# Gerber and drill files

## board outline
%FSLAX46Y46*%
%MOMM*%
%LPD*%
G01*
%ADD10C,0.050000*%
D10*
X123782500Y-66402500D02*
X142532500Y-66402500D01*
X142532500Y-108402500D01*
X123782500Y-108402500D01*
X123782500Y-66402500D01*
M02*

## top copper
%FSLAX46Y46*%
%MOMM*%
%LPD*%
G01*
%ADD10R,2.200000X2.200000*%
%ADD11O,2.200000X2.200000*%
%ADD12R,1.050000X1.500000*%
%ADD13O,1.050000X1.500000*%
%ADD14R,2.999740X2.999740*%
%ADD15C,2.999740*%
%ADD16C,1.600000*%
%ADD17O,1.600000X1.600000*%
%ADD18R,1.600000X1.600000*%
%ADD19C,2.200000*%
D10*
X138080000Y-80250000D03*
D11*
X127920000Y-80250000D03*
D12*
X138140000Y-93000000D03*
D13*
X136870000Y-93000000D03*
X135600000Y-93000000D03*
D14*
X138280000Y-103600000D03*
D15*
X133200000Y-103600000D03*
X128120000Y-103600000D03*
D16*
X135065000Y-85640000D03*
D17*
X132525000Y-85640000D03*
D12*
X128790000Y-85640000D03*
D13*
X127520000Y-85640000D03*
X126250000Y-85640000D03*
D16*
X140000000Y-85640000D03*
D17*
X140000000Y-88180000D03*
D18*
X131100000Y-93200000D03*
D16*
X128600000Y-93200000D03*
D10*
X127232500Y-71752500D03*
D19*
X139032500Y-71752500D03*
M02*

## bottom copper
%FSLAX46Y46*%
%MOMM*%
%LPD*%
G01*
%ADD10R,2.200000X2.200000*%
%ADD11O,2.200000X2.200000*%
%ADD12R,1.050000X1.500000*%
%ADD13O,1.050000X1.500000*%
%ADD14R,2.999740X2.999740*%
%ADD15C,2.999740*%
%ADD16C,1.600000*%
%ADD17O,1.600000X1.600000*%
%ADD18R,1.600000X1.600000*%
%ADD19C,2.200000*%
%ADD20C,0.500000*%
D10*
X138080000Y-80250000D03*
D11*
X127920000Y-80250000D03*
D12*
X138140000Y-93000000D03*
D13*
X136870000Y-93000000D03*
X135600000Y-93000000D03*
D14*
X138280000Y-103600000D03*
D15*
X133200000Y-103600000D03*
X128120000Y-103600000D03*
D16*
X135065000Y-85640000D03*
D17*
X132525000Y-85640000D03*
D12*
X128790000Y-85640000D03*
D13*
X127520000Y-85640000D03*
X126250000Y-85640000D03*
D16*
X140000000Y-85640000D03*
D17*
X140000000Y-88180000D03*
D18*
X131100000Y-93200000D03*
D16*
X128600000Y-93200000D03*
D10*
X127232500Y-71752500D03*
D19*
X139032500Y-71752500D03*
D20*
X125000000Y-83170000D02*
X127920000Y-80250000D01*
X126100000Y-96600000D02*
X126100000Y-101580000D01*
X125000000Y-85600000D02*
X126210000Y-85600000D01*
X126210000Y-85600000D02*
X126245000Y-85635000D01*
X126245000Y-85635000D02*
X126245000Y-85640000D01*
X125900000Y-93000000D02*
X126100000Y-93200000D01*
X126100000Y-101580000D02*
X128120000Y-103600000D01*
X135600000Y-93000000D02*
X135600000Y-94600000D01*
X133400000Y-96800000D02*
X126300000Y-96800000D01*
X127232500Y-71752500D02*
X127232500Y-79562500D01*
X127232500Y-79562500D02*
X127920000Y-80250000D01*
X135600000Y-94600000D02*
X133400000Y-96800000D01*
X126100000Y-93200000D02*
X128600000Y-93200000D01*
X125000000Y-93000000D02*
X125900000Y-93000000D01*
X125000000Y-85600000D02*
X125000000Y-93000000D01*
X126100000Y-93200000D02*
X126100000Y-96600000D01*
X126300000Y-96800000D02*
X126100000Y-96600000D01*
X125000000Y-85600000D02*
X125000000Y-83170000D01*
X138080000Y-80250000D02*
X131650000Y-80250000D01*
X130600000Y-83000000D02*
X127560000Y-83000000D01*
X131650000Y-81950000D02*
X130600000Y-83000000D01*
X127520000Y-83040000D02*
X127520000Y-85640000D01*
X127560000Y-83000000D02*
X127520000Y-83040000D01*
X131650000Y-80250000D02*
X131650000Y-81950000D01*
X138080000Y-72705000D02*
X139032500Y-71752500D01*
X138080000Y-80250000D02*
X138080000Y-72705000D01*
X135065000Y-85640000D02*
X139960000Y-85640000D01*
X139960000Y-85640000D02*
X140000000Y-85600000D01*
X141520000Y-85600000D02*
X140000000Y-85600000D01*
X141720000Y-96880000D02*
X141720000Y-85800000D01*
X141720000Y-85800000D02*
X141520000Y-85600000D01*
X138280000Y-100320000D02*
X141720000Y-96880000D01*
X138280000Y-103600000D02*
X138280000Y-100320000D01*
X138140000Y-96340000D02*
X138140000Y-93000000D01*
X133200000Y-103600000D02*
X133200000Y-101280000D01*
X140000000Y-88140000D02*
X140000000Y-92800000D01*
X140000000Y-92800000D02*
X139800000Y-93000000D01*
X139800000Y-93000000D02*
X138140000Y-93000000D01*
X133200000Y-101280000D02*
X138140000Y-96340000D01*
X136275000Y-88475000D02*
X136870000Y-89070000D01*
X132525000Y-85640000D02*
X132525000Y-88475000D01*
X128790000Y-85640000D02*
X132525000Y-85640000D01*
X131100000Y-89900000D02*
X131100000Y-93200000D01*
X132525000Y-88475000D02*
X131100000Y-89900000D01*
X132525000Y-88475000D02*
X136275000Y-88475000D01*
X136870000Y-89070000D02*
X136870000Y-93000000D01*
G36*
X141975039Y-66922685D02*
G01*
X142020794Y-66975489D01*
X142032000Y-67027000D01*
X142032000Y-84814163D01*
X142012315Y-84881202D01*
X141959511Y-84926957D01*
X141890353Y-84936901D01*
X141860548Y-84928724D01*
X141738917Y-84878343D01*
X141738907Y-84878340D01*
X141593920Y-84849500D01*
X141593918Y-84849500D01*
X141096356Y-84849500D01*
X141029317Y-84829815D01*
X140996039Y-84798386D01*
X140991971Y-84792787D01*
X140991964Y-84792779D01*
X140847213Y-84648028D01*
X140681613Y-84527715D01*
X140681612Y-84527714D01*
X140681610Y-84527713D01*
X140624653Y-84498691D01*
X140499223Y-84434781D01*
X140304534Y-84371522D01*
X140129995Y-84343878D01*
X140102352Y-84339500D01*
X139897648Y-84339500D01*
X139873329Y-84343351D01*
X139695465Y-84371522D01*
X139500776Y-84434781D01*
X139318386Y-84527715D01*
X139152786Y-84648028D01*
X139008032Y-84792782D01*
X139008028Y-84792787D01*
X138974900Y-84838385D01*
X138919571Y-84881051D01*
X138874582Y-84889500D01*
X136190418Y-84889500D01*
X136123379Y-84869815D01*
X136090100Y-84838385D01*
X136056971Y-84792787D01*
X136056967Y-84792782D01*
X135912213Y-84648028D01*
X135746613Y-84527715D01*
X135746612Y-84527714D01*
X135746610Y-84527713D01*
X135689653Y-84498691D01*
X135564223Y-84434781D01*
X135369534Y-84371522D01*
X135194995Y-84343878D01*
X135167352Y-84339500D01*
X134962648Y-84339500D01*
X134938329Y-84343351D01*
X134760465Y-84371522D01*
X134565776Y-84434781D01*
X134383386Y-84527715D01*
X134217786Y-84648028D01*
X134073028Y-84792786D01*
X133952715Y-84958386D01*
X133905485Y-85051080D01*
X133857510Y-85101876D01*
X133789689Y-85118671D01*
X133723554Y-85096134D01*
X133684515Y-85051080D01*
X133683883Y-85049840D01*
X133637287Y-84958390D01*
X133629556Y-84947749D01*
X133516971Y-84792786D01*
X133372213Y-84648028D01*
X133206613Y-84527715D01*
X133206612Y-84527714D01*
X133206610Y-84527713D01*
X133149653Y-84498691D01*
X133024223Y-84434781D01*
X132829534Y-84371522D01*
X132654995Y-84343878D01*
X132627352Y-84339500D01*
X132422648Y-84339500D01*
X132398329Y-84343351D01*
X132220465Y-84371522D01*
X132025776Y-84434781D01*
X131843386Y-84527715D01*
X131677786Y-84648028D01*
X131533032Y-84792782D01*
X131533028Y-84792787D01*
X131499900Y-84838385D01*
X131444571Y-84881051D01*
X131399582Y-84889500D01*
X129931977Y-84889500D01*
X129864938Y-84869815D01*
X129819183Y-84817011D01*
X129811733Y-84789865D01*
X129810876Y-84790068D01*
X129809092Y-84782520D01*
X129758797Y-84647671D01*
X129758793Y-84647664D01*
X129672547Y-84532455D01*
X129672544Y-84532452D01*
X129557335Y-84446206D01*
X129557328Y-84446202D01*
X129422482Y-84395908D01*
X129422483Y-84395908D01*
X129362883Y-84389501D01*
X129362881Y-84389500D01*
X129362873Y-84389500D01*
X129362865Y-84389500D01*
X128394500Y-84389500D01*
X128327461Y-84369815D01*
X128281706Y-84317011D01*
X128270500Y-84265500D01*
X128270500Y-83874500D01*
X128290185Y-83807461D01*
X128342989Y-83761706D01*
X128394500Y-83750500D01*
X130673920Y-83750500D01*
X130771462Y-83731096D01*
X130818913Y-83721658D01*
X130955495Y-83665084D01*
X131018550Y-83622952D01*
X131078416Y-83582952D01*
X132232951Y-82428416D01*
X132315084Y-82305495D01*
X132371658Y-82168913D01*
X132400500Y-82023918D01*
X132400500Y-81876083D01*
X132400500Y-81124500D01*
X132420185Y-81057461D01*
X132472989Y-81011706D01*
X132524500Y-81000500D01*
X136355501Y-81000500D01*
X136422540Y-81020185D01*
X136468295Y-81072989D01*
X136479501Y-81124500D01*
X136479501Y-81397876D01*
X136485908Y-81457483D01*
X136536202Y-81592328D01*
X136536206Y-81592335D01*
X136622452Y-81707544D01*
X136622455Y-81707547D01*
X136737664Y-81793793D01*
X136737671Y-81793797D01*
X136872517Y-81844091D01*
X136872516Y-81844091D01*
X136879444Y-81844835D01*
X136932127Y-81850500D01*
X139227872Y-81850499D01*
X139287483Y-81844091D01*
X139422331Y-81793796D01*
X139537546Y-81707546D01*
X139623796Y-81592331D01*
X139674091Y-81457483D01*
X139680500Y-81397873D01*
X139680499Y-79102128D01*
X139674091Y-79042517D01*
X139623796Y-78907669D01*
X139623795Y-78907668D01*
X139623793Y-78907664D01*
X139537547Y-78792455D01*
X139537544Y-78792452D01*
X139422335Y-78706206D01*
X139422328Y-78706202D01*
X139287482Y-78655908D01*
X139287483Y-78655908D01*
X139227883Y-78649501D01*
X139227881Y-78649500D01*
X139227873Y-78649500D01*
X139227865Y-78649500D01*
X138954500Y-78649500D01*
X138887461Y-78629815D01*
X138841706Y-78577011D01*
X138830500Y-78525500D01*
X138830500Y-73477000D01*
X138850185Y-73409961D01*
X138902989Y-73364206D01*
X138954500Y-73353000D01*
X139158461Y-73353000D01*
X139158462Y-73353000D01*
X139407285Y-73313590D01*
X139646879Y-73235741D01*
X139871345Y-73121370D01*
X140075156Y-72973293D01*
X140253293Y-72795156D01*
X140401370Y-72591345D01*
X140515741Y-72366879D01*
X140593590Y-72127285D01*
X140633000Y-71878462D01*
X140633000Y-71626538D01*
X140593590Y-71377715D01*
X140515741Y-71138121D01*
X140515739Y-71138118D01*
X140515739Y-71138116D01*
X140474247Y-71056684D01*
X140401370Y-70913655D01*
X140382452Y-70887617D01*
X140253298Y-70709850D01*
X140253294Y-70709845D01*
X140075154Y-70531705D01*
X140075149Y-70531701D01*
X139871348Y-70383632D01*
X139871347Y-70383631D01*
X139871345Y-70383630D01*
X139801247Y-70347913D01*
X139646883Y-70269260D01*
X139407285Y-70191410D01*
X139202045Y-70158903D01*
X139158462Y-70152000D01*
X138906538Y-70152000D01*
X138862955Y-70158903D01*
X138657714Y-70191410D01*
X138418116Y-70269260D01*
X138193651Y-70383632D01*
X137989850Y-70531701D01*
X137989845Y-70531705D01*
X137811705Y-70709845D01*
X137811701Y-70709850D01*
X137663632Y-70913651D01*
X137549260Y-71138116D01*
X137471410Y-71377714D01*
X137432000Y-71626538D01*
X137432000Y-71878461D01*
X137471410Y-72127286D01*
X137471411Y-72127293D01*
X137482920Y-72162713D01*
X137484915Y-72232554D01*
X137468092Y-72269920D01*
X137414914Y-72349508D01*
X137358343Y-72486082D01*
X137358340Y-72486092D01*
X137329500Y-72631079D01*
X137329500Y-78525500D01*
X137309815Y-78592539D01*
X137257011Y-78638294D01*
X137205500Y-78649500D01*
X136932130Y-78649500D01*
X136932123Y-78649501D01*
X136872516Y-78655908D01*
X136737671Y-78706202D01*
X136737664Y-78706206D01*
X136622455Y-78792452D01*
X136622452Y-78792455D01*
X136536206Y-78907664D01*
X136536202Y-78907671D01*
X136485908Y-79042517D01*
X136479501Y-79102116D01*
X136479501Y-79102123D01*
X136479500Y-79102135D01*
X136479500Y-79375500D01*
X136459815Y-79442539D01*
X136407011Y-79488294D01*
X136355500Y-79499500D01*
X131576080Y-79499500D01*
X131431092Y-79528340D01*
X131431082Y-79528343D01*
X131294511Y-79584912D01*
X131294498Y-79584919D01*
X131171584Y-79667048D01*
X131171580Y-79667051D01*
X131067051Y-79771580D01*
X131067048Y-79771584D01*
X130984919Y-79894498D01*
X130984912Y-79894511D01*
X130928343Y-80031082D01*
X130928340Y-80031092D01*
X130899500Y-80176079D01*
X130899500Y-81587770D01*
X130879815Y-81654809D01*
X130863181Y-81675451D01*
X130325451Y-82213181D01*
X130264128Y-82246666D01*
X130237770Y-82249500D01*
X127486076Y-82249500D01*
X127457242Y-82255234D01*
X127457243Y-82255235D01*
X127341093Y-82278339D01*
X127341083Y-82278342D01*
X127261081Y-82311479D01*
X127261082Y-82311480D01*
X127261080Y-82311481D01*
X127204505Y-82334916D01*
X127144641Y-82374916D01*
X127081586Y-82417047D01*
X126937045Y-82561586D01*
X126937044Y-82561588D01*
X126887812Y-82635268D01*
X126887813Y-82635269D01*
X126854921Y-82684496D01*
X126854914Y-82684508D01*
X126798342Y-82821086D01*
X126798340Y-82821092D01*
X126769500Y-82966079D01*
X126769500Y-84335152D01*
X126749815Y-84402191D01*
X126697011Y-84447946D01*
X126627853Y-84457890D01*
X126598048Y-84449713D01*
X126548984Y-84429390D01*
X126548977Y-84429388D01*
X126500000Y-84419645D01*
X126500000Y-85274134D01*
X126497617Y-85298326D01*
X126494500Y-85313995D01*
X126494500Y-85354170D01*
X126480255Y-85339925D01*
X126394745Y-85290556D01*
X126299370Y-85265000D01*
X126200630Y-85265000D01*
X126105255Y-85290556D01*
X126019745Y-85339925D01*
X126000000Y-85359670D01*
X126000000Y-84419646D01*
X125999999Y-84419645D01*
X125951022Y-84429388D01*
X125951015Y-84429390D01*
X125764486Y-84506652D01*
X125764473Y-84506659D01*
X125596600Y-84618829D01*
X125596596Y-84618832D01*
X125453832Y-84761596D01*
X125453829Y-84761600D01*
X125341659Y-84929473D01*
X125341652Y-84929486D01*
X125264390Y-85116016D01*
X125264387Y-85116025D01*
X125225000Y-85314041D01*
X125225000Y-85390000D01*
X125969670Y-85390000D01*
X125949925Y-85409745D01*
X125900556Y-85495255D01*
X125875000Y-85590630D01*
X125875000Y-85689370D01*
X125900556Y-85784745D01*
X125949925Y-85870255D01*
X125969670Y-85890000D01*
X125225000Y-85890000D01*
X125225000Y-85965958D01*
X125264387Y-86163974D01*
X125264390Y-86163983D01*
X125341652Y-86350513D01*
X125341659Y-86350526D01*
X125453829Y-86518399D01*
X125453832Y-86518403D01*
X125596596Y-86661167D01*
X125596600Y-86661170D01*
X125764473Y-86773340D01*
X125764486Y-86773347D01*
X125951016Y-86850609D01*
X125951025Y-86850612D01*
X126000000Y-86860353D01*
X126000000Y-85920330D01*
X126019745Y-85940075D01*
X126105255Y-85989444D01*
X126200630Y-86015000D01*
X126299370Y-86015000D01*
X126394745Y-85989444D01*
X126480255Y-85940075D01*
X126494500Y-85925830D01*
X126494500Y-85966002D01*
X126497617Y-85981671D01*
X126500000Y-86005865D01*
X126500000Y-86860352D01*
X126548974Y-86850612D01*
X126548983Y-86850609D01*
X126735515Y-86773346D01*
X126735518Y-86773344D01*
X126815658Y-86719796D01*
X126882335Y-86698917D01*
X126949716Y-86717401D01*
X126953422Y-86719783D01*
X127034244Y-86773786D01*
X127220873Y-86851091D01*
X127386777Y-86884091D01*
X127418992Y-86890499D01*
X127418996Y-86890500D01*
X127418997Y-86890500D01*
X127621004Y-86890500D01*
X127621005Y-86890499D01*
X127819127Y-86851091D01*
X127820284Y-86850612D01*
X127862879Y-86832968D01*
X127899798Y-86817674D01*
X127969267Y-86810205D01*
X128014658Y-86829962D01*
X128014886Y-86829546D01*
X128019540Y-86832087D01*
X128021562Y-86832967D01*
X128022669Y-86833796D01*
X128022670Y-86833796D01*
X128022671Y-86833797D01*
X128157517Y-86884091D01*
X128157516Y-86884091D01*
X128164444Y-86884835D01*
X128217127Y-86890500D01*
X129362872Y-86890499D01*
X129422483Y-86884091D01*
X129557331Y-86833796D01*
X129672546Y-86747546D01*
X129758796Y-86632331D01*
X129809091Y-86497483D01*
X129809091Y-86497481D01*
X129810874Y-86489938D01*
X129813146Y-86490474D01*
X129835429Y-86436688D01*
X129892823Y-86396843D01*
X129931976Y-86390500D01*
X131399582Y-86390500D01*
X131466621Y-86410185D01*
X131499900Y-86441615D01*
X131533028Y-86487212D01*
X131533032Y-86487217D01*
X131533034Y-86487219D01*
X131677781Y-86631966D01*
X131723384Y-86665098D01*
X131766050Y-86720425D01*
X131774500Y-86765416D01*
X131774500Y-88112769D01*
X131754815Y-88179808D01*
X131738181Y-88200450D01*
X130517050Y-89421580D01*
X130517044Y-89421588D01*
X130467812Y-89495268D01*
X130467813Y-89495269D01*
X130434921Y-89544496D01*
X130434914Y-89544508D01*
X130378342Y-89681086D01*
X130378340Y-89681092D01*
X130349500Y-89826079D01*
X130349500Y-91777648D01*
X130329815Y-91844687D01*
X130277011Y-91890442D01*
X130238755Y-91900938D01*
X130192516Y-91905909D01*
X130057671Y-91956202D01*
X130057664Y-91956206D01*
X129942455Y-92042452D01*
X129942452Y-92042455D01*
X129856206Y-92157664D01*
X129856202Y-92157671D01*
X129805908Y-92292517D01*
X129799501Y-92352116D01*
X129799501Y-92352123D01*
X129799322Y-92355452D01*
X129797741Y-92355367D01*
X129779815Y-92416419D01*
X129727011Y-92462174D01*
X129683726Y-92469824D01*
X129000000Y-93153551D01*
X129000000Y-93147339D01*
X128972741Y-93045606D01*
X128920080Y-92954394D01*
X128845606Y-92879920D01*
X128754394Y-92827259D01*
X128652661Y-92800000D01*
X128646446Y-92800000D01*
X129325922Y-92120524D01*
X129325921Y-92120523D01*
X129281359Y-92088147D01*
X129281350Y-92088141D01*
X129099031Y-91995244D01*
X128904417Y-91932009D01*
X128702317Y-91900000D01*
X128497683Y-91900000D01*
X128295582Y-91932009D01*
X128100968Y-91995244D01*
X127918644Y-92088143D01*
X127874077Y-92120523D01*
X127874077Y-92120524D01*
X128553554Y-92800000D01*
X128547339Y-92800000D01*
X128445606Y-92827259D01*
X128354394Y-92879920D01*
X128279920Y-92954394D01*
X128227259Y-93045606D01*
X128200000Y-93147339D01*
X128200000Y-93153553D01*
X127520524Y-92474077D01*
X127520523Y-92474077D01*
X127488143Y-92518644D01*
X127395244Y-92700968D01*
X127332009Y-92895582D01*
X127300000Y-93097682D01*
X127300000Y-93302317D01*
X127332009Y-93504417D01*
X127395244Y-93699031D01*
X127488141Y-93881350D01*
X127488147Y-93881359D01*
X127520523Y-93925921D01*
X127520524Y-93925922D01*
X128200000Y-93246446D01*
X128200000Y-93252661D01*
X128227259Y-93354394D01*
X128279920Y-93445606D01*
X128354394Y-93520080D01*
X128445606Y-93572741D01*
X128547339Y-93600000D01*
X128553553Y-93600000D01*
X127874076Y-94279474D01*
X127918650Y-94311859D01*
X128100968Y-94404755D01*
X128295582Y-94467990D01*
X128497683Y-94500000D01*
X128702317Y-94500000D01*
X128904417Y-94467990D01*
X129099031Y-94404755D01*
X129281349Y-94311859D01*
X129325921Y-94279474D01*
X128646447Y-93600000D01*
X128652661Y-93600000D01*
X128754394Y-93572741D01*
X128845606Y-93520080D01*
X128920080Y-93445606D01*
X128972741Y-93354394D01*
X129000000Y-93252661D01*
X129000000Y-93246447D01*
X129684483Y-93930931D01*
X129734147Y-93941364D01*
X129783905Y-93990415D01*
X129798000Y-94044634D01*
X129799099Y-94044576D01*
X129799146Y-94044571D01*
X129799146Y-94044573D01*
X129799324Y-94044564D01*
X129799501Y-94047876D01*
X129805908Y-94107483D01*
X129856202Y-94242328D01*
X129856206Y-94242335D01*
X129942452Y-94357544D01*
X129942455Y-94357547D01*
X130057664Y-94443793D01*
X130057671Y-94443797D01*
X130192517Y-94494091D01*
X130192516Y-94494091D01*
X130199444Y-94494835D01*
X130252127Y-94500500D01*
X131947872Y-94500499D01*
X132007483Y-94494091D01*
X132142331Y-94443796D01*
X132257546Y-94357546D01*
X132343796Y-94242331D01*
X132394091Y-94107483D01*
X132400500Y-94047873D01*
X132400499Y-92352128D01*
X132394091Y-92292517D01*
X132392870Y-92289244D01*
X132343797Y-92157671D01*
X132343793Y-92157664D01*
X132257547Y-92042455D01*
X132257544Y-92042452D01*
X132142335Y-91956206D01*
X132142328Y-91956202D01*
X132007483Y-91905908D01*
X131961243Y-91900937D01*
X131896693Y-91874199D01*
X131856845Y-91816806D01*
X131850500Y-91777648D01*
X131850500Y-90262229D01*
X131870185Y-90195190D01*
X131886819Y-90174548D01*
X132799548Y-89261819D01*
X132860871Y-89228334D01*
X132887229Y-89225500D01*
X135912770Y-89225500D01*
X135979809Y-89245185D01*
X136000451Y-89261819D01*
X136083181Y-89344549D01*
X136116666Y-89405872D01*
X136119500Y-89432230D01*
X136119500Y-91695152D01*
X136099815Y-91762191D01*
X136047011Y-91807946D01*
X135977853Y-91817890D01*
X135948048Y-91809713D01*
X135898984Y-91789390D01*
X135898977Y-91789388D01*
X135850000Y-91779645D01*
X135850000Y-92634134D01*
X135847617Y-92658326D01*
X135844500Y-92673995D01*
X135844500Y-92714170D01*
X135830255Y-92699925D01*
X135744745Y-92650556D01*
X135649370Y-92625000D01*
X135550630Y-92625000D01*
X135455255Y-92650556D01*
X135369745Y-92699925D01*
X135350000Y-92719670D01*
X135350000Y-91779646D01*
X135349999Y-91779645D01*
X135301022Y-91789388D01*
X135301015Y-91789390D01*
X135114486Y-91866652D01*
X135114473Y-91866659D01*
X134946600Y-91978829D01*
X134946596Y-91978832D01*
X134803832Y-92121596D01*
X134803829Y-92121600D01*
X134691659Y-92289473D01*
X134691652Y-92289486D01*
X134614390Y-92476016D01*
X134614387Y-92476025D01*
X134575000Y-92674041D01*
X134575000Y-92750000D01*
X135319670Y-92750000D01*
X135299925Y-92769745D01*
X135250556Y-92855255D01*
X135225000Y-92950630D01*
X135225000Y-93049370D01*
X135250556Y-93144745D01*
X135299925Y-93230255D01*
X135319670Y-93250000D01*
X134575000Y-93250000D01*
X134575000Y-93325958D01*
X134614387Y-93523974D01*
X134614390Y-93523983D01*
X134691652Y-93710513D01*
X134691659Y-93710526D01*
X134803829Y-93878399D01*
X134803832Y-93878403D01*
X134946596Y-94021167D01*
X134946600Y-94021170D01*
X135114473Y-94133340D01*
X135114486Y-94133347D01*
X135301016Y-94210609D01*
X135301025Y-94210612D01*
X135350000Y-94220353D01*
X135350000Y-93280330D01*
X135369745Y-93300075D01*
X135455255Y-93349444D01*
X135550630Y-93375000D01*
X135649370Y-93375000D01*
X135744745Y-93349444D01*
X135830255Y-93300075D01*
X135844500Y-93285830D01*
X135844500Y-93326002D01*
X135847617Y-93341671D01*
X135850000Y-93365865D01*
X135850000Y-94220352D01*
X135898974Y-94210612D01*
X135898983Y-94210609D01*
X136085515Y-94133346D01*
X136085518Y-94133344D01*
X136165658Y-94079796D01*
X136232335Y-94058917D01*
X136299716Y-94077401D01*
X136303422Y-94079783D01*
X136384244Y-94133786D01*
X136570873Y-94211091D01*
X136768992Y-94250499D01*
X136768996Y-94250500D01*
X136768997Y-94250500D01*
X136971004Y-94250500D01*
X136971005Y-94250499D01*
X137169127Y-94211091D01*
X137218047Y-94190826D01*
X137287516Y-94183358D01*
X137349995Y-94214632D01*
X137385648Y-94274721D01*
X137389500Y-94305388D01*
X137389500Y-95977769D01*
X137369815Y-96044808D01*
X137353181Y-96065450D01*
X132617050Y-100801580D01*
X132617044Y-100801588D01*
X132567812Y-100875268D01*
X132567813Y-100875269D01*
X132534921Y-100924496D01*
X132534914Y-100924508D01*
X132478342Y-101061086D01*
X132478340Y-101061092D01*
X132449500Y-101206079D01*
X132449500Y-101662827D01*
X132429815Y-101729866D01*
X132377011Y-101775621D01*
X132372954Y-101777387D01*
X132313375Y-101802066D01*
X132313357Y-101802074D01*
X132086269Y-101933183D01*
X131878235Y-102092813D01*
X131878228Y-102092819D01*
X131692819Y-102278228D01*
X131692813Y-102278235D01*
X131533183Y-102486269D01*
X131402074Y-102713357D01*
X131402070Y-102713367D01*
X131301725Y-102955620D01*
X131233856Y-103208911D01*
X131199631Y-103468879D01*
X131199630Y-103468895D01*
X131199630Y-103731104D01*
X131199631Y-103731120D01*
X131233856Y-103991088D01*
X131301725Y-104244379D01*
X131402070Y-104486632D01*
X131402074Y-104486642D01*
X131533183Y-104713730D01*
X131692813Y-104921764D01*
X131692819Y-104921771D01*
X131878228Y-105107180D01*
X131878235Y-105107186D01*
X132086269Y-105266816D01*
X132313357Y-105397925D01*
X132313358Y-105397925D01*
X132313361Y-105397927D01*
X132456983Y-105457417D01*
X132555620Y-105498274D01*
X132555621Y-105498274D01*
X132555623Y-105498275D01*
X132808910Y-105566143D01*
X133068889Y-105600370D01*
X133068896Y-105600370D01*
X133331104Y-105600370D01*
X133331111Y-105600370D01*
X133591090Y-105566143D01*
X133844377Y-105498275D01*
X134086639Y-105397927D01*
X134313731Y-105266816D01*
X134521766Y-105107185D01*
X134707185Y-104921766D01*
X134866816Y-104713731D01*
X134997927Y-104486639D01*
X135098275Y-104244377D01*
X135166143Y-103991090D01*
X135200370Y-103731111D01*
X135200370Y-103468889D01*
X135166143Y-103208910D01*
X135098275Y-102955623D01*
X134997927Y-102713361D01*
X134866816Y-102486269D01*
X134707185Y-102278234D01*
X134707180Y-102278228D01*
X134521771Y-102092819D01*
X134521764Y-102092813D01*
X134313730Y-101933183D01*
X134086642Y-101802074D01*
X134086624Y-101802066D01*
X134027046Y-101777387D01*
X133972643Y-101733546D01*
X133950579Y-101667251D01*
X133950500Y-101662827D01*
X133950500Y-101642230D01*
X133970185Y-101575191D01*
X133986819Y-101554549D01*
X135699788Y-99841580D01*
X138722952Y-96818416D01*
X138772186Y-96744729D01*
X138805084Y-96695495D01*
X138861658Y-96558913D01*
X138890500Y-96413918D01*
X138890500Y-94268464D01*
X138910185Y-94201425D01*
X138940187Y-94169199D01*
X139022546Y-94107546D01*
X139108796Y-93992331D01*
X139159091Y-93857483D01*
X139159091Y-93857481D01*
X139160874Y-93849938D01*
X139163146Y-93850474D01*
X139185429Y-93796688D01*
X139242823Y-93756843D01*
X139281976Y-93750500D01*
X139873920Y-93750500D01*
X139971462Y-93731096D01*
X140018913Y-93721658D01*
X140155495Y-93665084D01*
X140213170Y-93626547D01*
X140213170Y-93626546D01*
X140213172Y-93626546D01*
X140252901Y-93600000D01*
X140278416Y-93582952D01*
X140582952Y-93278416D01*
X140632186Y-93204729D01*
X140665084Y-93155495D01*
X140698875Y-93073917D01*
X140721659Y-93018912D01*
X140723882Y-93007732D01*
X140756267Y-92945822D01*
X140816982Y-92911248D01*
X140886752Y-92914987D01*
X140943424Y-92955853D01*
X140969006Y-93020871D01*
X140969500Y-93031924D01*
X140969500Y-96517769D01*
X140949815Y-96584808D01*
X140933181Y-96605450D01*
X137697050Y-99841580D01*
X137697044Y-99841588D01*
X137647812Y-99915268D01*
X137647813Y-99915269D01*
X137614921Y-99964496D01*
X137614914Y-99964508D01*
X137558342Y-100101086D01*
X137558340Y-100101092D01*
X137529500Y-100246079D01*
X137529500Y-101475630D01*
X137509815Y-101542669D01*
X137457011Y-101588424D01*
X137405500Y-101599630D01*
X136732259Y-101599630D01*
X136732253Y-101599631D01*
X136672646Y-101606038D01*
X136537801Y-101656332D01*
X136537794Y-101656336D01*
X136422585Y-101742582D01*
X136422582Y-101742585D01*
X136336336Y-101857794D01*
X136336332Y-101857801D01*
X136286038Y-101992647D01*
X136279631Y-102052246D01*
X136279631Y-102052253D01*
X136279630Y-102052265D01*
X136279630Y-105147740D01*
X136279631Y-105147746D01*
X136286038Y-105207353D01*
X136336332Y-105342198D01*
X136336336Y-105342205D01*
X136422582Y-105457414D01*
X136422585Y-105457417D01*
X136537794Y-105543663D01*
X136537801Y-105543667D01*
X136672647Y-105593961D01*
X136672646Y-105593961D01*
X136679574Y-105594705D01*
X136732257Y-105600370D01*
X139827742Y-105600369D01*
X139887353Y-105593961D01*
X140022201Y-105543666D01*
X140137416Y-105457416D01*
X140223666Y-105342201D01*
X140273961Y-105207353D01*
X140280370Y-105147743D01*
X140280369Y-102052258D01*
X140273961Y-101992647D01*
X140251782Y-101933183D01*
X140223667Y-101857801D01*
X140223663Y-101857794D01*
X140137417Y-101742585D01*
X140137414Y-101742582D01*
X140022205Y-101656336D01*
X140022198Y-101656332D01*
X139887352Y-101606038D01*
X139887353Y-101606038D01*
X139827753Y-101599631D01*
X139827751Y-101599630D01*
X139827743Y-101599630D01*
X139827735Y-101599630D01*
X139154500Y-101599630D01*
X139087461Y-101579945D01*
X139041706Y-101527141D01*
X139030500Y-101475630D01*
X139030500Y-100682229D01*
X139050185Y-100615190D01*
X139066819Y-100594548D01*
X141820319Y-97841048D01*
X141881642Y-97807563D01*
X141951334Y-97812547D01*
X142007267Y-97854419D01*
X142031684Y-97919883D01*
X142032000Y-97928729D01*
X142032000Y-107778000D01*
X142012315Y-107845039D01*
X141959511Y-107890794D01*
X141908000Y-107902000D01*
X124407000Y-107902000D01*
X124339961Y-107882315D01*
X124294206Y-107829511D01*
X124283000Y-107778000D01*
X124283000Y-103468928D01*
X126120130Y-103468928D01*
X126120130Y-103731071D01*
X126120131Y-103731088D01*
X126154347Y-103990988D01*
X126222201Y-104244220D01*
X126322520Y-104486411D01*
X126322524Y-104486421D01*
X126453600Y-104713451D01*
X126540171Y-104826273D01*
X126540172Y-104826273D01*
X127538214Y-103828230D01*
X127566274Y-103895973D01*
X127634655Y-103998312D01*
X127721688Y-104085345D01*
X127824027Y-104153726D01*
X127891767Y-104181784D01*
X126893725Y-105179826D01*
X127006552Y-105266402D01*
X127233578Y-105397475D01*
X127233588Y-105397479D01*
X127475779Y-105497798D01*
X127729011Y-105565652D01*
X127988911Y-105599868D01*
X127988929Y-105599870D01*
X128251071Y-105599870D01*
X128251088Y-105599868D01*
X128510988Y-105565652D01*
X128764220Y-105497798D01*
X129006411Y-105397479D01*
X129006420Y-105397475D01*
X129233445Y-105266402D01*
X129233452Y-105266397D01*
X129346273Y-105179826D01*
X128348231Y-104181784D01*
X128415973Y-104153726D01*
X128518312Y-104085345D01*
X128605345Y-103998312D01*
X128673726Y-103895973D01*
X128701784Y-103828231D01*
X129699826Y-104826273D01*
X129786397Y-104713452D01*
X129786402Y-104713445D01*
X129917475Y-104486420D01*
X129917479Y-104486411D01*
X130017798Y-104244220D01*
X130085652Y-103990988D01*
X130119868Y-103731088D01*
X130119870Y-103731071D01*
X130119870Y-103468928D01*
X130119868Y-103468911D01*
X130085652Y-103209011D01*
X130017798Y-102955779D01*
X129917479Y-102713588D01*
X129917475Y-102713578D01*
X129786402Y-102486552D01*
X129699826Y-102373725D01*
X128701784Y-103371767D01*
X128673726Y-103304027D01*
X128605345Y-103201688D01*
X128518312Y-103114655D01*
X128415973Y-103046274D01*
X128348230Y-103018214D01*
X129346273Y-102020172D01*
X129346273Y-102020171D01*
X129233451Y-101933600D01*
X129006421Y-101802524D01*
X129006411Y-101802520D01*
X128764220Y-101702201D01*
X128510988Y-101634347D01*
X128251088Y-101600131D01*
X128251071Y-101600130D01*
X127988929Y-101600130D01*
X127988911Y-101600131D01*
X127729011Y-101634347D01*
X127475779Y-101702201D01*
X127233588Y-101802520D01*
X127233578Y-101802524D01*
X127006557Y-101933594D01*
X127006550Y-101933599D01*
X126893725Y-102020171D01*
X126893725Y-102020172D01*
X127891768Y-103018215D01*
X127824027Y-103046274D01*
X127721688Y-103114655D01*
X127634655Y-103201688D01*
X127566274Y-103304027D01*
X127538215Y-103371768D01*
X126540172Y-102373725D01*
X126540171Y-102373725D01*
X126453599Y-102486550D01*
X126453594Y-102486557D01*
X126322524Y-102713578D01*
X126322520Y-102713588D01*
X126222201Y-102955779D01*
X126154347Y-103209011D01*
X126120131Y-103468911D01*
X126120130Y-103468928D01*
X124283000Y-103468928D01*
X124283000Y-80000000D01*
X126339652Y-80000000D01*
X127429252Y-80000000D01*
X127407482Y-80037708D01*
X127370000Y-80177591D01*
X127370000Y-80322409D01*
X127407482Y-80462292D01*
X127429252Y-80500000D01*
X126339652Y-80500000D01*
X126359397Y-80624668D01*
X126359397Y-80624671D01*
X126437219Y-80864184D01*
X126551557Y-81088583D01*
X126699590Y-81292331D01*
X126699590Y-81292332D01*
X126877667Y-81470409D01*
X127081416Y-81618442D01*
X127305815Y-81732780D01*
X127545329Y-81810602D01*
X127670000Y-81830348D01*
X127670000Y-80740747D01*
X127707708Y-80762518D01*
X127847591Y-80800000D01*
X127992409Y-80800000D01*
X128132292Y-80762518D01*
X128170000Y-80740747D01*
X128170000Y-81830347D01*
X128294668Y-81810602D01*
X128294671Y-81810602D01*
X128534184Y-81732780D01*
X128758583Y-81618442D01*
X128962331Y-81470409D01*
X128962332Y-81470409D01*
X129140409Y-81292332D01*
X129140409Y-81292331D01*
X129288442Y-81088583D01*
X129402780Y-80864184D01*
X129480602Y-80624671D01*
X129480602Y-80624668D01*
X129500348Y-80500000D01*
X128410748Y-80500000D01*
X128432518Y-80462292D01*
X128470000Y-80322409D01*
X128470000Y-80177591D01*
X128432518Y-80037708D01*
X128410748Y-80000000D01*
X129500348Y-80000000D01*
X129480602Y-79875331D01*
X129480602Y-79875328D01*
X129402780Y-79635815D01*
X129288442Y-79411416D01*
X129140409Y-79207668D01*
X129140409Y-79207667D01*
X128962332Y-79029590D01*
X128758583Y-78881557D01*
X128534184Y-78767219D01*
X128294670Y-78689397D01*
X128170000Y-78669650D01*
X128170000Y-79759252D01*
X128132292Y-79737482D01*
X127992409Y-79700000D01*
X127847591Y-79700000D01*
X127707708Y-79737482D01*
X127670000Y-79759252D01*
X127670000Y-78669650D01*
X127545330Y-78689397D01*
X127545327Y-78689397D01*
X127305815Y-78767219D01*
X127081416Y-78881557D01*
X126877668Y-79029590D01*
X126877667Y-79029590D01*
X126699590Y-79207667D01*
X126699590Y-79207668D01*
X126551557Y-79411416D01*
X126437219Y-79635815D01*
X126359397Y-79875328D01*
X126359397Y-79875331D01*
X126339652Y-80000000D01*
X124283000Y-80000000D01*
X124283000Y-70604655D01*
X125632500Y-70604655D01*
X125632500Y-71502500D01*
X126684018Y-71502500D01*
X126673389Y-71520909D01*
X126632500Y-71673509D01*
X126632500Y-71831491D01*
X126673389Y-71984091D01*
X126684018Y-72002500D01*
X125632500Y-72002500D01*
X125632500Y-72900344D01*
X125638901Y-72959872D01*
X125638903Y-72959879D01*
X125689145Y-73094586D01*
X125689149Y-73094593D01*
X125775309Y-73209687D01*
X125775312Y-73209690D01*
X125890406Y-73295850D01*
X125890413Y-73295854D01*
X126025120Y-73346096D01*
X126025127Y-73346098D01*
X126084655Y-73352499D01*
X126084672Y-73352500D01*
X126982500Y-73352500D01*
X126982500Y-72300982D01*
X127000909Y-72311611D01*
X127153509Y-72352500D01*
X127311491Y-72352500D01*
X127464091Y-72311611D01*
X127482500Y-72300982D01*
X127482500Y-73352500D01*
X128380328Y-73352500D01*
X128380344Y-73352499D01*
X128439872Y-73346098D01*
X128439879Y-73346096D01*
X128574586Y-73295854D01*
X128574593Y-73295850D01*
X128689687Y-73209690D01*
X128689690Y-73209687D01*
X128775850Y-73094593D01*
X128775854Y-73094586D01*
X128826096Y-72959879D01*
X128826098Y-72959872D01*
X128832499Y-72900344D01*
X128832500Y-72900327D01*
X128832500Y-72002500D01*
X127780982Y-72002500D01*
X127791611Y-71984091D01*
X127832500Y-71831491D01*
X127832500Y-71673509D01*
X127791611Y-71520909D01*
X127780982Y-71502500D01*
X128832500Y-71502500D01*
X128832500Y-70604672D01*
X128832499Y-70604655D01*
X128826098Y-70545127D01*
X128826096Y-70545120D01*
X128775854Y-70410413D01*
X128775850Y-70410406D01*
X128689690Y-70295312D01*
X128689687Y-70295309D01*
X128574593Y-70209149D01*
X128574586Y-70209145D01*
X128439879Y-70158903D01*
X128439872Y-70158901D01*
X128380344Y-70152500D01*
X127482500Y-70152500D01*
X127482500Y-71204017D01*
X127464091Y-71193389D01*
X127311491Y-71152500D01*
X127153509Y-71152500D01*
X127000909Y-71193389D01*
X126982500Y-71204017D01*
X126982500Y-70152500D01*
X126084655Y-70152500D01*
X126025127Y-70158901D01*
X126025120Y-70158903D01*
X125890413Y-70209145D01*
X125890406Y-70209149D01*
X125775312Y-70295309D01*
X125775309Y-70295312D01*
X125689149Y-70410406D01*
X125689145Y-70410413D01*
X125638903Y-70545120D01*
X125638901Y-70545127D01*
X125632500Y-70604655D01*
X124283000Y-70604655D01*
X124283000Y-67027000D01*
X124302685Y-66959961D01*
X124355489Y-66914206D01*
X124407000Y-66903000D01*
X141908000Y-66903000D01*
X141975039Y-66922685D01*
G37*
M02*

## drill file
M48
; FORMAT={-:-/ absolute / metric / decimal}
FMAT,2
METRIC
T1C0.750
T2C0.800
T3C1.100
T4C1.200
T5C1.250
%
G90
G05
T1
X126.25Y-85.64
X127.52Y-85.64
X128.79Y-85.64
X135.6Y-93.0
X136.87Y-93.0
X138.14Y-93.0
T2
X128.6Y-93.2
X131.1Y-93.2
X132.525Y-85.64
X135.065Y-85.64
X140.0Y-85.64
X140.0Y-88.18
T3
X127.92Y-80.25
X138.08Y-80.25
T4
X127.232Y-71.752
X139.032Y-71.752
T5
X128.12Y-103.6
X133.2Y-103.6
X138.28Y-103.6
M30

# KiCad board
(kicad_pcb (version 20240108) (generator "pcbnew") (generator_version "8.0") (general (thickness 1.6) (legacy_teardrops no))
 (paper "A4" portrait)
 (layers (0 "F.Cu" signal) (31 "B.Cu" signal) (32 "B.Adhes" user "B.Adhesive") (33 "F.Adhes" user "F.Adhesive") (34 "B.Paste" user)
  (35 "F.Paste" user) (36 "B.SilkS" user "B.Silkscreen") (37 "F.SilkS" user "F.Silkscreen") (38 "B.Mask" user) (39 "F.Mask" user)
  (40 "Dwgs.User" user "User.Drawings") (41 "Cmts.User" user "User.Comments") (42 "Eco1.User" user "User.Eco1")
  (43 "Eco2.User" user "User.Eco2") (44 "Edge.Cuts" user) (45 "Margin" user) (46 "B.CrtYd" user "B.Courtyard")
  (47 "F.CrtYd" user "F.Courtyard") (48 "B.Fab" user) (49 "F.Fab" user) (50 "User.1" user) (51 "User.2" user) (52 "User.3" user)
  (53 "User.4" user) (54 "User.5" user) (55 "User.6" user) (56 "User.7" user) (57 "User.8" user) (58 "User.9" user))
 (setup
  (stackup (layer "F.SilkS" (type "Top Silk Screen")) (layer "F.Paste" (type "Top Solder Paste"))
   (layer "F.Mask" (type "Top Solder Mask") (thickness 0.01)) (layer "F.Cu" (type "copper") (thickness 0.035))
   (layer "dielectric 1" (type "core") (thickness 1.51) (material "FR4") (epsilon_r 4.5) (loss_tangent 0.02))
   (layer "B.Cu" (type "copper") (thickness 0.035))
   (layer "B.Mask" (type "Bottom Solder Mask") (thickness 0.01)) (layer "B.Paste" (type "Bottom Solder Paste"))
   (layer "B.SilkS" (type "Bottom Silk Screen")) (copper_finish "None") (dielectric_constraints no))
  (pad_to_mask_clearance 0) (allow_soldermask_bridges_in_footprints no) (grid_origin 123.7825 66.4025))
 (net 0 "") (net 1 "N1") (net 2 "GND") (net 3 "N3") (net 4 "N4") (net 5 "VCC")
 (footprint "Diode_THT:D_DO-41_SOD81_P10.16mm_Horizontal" (layer "F.Cu") (at 138.08 80.25 180)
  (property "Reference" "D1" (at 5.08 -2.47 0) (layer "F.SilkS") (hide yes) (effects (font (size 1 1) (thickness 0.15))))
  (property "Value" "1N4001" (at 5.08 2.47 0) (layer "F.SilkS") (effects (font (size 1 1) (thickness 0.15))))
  (pad "1" thru_hole rect (at 0 0 180) (size 2.2 2.2) (drill 1.1) (layers "*.Cu" "*.Mask") (remove_unused_layers no) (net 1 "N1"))
  (pad "2" thru_hole oval (at 10.16 0 180) (size 2.2 2.2) (drill 1.1) (layers "*.Cu" "*.Mask") (remove_unused_layers no) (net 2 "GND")))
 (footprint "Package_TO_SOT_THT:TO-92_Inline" (layer "F.Cu") (at 138.14 93 180)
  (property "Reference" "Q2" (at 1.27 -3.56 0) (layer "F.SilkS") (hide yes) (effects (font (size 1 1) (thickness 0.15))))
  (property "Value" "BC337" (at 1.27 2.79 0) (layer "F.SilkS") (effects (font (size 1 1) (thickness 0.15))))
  (pad "1" thru_hole rect (at 0 0 180) (size 1.05 1.5) (drill 0.75) (layers "*.Cu" "*.Mask") (remove_unused_layers no) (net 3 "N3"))
  (pad "2" thru_hole oval (at 1.27 0 180) (size 1.05 1.5) (drill 0.75) (layers "*.Cu" "*.Mask") (remove_unused_layers no) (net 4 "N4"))
  (pad "3" thru_hole oval (at 2.54 0 180) (size 1.05 1.5) (drill 0.75) (layers "*.Cu" "*.Mask") (remove_unused_layers no) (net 2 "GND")))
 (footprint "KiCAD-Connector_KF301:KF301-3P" (layer "F.Cu") (at 133.2 103.6 180)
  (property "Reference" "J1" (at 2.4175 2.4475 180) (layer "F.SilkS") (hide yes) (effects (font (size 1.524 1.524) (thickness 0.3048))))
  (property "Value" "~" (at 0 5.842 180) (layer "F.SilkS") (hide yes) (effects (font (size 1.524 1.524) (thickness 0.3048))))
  (pad "1" thru_hole rect (at -5.08 0 180) (size 2.99974 2.99974) (drill 1.24968) (layers "*.Cu" "*.Mask") (remove_unused_layers no)
   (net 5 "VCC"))
  (pad "2" thru_hole circle (at 0 0 180) (size 2.99974 2.99974) (drill 1.24968) (layers "*.Cu" "*.Mask") (remove_unused_layers no)
   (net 3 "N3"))
  (pad "3" thru_hole circle (at 5.08 0 180) (size 2.99974 2.99974) (drill 1.24968) (layers "*.Cu" "*.Mask") (remove_unused_layers no)
   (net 2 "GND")))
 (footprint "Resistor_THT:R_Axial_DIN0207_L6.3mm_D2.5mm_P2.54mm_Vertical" (layer "F.Cu") (at 135.065 85.64 180)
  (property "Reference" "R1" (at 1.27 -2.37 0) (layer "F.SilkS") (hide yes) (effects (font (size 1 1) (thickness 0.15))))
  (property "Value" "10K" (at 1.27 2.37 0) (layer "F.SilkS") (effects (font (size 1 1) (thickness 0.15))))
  (pad "1" thru_hole circle (at 0 0 180) (size 1.6 1.6) (drill 0.8) (layers "*.Cu" "*.Mask") (remove_unused_layers no) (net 5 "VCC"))
  (pad "2" thru_hole oval (at 2.54 0 180) (size 1.6 1.6) (drill 0.8) (layers "*.Cu" "*.Mask") (remove_unused_layers no) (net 4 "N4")))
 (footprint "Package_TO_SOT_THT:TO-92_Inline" (layer "F.Cu") (at 128.79 85.64 180)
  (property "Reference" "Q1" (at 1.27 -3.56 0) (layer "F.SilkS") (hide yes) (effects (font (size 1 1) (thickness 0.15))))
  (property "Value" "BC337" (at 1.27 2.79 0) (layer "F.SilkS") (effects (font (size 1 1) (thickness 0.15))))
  (pad "1" thru_hole rect (at 0 0 180) (size 1.05 1.5) (drill 0.75) (layers "*.Cu" "*.Mask") (remove_unused_layers no) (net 4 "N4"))
  (pad "2" thru_hole oval (at 1.27 0 180) (size 1.05 1.5) (drill 0.75) (layers "*.Cu" "*.Mask") (remove_unused_layers no) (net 1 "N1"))
  (pad "3" thru_hole oval (at 2.54 0 180) (size 1.05 1.5) (drill 0.75) (layers "*.Cu" "*.Mask") (remove_unused_layers no) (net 2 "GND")))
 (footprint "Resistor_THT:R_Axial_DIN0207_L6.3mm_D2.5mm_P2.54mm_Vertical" (layer "F.Cu") (at 140 85.64 -90)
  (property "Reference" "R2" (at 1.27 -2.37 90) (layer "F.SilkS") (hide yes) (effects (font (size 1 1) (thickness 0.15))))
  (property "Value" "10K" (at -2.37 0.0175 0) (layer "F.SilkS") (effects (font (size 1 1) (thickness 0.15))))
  (pad "1" thru_hole circle (at 0 0 270) (size 1.6 1.6) (drill 0.8) (layers "*.Cu" "*.Mask") (remove_unused_layers no) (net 5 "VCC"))
  (pad "2" thru_hole oval (at 2.54 0 270) (size 1.6 1.6) (drill 0.8) (layers "*.Cu" "*.Mask") (remove_unused_layers no) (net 3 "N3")))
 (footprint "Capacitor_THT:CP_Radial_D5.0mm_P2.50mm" (layer "F.Cu") (at 131.1 93.2 180)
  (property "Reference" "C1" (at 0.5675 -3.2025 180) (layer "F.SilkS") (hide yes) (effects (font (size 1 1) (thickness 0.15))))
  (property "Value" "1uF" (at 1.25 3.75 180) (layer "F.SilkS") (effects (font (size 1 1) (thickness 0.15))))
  (pad "1" thru_hole rect (at 0 0 180) (size 1.6 1.6) (drill 0.8) (layers "*.Cu" "*.Mask") (remove_unused_layers no) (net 4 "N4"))
  (pad "2" thru_hole circle (at 2.5 0 180) (size 1.6 1.6) (drill 0.8) (layers "*.Cu" "*.Mask") (remove_unused_layers no) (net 2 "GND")))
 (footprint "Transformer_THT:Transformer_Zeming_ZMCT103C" (layer "F.Cu") (at 127.2325 71.7525)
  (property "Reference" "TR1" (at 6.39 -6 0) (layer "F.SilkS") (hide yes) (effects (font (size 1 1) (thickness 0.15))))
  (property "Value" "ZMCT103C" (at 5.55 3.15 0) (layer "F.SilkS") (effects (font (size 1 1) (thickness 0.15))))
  (pad "1" thru_hole rect (at 0 0) (size 2.2 2.2) (drill 1.2) (layers "*.Cu" "*.Mask") (remove_unused_layers no) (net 2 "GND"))
  (pad "2" thru_hole circle (at 11.8 0) (size 2.2 2.2) (drill 1.2) (layers "*.Cu" "*.Mask") (remove_unused_layers no) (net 1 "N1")))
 (gr_rect (start 123.7825 66.4025) (end 142.5325 108.4025) (stroke (width 0.05) (type default)) (fill none) (layer "Edge.Cuts"))
 (segment (start 125 83.17) (end 127.92 80.25) (width 0.5) (layer "B.Cu") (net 2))
 (segment (start 126.1 96.6) (end 126.1 101.58) (width 0.5) (layer "B.Cu") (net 2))
 (segment (start 125 85.6) (end 126.21 85.6) (width 0.5) (layer "B.Cu") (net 2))
 (segment (start 126.21 85.6) (end 126.245 85.635) (width 0.5) (layer "B.Cu") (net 2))
 (segment (start 126.245 85.635) (end 126.245 85.64) (width 0.5) (layer "B.Cu") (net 2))
 (segment (start 125.9 93) (end 126.1 93.2) (width 0.5) (layer "B.Cu") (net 2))
 (segment (start 126.1 101.58) (end 128.12 103.6) (width 0.5) (layer "B.Cu") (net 2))
 (segment (start 135.6 93) (end 135.6 94.6) (width 0.5) (layer "B.Cu") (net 2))
 (segment (start 133.4 96.8) (end 126.3 96.8) (width 0.5) (layer "B.Cu") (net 2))
 (segment (start 127.2325 71.7525) (end 127.2325 79.5625) (width 0.5) (layer "B.Cu") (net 2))
 (segment (start 127.2325 79.5625) (end 127.92 80.25) (width 0.5) (layer "B.Cu") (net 2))
 (segment (start 135.6 94.6) (end 133.4 96.8) (width 0.5) (layer "B.Cu") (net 2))
 (segment (start 126.1 93.2) (end 128.6 93.2) (width 0.5) (layer "B.Cu") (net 2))
 (segment (start 125 93) (end 125.9 93) (width 0.5) (layer "B.Cu") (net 2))
 (segment (start 125 85.6) (end 125 93) (width 0.5) (layer "B.Cu") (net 2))
 (segment (start 126.1 93.2) (end 126.1 96.6) (width 0.5) (layer "B.Cu") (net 2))
 (segment (start 126.3 96.8) (end 126.1 96.6) (width 0.5) (layer "B.Cu") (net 2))
 (segment (start 125 85.6) (end 125 83.17) (width 0.5) (layer "B.Cu") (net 2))
 (segment (start 138.08 80.25) (end 131.65 80.25) (width 0.5) (layer "B.Cu") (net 1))
 (segment (start 130.6 83) (end 127.56 83) (width 0.5) (layer "B.Cu") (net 1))
 (segment (start 131.65 81.95) (end 130.6 83) (width 0.5) (layer "B.Cu") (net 1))
 (segment (start 127.52 83.04) (end 127.52 85.64) (width 0.5) (layer "B.Cu") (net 1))
 (segment (start 127.56 83) (end 127.52 83.04) (width 0.5) (layer "B.Cu") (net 1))
 (segment (start 131.65 80.25) (end 131.65 81.95) (width 0.5) (layer "B.Cu") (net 1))
 (segment (start 138.08 72.705) (end 139.0325 71.7525) (width 0.5) (layer "B.Cu") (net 1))
 (segment (start 138.08 80.25) (end 138.08 72.705) (width 0.5) (layer "B.Cu") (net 1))
 (segment (start 135.065 85.64) (end 139.96 85.64) (width 0.5) (layer "B.Cu") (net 5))
 (segment (start 139.96 85.64) (end 140 85.6) (width 0.5) (layer "B.Cu") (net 5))
 (segment (start 141.52 85.6) (end 140 85.6) (width 0.5) (layer "B.Cu") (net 5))
 (segment (start 141.72 96.88) (end 141.72 85.8) (width 0.5) (layer "B.Cu") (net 5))
 (segment (start 141.72 85.8) (end 141.52 85.6) (width 0.5) (layer "B.Cu") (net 5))
 (segment (start 138.28 100.32) (end 141.72 96.88) (width 0.5) (layer "B.Cu") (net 5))
 (segment (start 138.28 103.6) (end 138.28 100.32) (width 0.5) (layer "B.Cu") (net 5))
 (segment (start 138.14 96.34) (end 138.14 93) (width 0.5) (layer "B.Cu") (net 3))
 (segment (start 133.2 103.6) (end 133.2 101.28) (width 0.5) (layer "B.Cu") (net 3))
 (segment (start 140 88.14) (end 140 92.8) (width 0.5) (layer "B.Cu") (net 3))
 (segment (start 140 92.8) (end 139.8 93) (width 0.5) (layer "B.Cu") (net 3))
 (segment (start 139.8 93) (end 138.14 93) (width 0.5) (layer "B.Cu") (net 3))
 (segment (start 133.2 101.28) (end 138.14 96.34) (width 0.5) (layer "B.Cu") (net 3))
 (segment (start 136.275 88.475) (end 136.87 89.07) (width 0.5) (layer "B.Cu") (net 4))
 (segment (start 132.525 85.64) (end 132.525 88.475) (width 0.5) (layer "B.Cu") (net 4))
 (segment (start 128.79 85.64) (end 132.525 85.64) (width 0.5) (layer "B.Cu") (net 4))
 (segment (start 131.1 89.9) (end 131.1 93.2) (width 0.5) (layer "B.Cu") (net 4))
 (segment (start 132.525 88.475) (end 131.1 89.9) (width 0.5) (layer "B.Cu") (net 4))
 (segment (start 132.525 88.475) (end 136.275 88.475) (width 0.5) (layer "B.Cu") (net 4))
 (segment (start 136.87 89.07) (end 136.87 93) (width 0.5) (layer "B.Cu") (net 4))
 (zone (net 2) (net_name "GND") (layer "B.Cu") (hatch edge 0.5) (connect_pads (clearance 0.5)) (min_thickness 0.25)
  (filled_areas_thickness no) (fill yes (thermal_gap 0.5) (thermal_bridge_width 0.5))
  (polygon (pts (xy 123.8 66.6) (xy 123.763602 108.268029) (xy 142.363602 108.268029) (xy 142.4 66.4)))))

